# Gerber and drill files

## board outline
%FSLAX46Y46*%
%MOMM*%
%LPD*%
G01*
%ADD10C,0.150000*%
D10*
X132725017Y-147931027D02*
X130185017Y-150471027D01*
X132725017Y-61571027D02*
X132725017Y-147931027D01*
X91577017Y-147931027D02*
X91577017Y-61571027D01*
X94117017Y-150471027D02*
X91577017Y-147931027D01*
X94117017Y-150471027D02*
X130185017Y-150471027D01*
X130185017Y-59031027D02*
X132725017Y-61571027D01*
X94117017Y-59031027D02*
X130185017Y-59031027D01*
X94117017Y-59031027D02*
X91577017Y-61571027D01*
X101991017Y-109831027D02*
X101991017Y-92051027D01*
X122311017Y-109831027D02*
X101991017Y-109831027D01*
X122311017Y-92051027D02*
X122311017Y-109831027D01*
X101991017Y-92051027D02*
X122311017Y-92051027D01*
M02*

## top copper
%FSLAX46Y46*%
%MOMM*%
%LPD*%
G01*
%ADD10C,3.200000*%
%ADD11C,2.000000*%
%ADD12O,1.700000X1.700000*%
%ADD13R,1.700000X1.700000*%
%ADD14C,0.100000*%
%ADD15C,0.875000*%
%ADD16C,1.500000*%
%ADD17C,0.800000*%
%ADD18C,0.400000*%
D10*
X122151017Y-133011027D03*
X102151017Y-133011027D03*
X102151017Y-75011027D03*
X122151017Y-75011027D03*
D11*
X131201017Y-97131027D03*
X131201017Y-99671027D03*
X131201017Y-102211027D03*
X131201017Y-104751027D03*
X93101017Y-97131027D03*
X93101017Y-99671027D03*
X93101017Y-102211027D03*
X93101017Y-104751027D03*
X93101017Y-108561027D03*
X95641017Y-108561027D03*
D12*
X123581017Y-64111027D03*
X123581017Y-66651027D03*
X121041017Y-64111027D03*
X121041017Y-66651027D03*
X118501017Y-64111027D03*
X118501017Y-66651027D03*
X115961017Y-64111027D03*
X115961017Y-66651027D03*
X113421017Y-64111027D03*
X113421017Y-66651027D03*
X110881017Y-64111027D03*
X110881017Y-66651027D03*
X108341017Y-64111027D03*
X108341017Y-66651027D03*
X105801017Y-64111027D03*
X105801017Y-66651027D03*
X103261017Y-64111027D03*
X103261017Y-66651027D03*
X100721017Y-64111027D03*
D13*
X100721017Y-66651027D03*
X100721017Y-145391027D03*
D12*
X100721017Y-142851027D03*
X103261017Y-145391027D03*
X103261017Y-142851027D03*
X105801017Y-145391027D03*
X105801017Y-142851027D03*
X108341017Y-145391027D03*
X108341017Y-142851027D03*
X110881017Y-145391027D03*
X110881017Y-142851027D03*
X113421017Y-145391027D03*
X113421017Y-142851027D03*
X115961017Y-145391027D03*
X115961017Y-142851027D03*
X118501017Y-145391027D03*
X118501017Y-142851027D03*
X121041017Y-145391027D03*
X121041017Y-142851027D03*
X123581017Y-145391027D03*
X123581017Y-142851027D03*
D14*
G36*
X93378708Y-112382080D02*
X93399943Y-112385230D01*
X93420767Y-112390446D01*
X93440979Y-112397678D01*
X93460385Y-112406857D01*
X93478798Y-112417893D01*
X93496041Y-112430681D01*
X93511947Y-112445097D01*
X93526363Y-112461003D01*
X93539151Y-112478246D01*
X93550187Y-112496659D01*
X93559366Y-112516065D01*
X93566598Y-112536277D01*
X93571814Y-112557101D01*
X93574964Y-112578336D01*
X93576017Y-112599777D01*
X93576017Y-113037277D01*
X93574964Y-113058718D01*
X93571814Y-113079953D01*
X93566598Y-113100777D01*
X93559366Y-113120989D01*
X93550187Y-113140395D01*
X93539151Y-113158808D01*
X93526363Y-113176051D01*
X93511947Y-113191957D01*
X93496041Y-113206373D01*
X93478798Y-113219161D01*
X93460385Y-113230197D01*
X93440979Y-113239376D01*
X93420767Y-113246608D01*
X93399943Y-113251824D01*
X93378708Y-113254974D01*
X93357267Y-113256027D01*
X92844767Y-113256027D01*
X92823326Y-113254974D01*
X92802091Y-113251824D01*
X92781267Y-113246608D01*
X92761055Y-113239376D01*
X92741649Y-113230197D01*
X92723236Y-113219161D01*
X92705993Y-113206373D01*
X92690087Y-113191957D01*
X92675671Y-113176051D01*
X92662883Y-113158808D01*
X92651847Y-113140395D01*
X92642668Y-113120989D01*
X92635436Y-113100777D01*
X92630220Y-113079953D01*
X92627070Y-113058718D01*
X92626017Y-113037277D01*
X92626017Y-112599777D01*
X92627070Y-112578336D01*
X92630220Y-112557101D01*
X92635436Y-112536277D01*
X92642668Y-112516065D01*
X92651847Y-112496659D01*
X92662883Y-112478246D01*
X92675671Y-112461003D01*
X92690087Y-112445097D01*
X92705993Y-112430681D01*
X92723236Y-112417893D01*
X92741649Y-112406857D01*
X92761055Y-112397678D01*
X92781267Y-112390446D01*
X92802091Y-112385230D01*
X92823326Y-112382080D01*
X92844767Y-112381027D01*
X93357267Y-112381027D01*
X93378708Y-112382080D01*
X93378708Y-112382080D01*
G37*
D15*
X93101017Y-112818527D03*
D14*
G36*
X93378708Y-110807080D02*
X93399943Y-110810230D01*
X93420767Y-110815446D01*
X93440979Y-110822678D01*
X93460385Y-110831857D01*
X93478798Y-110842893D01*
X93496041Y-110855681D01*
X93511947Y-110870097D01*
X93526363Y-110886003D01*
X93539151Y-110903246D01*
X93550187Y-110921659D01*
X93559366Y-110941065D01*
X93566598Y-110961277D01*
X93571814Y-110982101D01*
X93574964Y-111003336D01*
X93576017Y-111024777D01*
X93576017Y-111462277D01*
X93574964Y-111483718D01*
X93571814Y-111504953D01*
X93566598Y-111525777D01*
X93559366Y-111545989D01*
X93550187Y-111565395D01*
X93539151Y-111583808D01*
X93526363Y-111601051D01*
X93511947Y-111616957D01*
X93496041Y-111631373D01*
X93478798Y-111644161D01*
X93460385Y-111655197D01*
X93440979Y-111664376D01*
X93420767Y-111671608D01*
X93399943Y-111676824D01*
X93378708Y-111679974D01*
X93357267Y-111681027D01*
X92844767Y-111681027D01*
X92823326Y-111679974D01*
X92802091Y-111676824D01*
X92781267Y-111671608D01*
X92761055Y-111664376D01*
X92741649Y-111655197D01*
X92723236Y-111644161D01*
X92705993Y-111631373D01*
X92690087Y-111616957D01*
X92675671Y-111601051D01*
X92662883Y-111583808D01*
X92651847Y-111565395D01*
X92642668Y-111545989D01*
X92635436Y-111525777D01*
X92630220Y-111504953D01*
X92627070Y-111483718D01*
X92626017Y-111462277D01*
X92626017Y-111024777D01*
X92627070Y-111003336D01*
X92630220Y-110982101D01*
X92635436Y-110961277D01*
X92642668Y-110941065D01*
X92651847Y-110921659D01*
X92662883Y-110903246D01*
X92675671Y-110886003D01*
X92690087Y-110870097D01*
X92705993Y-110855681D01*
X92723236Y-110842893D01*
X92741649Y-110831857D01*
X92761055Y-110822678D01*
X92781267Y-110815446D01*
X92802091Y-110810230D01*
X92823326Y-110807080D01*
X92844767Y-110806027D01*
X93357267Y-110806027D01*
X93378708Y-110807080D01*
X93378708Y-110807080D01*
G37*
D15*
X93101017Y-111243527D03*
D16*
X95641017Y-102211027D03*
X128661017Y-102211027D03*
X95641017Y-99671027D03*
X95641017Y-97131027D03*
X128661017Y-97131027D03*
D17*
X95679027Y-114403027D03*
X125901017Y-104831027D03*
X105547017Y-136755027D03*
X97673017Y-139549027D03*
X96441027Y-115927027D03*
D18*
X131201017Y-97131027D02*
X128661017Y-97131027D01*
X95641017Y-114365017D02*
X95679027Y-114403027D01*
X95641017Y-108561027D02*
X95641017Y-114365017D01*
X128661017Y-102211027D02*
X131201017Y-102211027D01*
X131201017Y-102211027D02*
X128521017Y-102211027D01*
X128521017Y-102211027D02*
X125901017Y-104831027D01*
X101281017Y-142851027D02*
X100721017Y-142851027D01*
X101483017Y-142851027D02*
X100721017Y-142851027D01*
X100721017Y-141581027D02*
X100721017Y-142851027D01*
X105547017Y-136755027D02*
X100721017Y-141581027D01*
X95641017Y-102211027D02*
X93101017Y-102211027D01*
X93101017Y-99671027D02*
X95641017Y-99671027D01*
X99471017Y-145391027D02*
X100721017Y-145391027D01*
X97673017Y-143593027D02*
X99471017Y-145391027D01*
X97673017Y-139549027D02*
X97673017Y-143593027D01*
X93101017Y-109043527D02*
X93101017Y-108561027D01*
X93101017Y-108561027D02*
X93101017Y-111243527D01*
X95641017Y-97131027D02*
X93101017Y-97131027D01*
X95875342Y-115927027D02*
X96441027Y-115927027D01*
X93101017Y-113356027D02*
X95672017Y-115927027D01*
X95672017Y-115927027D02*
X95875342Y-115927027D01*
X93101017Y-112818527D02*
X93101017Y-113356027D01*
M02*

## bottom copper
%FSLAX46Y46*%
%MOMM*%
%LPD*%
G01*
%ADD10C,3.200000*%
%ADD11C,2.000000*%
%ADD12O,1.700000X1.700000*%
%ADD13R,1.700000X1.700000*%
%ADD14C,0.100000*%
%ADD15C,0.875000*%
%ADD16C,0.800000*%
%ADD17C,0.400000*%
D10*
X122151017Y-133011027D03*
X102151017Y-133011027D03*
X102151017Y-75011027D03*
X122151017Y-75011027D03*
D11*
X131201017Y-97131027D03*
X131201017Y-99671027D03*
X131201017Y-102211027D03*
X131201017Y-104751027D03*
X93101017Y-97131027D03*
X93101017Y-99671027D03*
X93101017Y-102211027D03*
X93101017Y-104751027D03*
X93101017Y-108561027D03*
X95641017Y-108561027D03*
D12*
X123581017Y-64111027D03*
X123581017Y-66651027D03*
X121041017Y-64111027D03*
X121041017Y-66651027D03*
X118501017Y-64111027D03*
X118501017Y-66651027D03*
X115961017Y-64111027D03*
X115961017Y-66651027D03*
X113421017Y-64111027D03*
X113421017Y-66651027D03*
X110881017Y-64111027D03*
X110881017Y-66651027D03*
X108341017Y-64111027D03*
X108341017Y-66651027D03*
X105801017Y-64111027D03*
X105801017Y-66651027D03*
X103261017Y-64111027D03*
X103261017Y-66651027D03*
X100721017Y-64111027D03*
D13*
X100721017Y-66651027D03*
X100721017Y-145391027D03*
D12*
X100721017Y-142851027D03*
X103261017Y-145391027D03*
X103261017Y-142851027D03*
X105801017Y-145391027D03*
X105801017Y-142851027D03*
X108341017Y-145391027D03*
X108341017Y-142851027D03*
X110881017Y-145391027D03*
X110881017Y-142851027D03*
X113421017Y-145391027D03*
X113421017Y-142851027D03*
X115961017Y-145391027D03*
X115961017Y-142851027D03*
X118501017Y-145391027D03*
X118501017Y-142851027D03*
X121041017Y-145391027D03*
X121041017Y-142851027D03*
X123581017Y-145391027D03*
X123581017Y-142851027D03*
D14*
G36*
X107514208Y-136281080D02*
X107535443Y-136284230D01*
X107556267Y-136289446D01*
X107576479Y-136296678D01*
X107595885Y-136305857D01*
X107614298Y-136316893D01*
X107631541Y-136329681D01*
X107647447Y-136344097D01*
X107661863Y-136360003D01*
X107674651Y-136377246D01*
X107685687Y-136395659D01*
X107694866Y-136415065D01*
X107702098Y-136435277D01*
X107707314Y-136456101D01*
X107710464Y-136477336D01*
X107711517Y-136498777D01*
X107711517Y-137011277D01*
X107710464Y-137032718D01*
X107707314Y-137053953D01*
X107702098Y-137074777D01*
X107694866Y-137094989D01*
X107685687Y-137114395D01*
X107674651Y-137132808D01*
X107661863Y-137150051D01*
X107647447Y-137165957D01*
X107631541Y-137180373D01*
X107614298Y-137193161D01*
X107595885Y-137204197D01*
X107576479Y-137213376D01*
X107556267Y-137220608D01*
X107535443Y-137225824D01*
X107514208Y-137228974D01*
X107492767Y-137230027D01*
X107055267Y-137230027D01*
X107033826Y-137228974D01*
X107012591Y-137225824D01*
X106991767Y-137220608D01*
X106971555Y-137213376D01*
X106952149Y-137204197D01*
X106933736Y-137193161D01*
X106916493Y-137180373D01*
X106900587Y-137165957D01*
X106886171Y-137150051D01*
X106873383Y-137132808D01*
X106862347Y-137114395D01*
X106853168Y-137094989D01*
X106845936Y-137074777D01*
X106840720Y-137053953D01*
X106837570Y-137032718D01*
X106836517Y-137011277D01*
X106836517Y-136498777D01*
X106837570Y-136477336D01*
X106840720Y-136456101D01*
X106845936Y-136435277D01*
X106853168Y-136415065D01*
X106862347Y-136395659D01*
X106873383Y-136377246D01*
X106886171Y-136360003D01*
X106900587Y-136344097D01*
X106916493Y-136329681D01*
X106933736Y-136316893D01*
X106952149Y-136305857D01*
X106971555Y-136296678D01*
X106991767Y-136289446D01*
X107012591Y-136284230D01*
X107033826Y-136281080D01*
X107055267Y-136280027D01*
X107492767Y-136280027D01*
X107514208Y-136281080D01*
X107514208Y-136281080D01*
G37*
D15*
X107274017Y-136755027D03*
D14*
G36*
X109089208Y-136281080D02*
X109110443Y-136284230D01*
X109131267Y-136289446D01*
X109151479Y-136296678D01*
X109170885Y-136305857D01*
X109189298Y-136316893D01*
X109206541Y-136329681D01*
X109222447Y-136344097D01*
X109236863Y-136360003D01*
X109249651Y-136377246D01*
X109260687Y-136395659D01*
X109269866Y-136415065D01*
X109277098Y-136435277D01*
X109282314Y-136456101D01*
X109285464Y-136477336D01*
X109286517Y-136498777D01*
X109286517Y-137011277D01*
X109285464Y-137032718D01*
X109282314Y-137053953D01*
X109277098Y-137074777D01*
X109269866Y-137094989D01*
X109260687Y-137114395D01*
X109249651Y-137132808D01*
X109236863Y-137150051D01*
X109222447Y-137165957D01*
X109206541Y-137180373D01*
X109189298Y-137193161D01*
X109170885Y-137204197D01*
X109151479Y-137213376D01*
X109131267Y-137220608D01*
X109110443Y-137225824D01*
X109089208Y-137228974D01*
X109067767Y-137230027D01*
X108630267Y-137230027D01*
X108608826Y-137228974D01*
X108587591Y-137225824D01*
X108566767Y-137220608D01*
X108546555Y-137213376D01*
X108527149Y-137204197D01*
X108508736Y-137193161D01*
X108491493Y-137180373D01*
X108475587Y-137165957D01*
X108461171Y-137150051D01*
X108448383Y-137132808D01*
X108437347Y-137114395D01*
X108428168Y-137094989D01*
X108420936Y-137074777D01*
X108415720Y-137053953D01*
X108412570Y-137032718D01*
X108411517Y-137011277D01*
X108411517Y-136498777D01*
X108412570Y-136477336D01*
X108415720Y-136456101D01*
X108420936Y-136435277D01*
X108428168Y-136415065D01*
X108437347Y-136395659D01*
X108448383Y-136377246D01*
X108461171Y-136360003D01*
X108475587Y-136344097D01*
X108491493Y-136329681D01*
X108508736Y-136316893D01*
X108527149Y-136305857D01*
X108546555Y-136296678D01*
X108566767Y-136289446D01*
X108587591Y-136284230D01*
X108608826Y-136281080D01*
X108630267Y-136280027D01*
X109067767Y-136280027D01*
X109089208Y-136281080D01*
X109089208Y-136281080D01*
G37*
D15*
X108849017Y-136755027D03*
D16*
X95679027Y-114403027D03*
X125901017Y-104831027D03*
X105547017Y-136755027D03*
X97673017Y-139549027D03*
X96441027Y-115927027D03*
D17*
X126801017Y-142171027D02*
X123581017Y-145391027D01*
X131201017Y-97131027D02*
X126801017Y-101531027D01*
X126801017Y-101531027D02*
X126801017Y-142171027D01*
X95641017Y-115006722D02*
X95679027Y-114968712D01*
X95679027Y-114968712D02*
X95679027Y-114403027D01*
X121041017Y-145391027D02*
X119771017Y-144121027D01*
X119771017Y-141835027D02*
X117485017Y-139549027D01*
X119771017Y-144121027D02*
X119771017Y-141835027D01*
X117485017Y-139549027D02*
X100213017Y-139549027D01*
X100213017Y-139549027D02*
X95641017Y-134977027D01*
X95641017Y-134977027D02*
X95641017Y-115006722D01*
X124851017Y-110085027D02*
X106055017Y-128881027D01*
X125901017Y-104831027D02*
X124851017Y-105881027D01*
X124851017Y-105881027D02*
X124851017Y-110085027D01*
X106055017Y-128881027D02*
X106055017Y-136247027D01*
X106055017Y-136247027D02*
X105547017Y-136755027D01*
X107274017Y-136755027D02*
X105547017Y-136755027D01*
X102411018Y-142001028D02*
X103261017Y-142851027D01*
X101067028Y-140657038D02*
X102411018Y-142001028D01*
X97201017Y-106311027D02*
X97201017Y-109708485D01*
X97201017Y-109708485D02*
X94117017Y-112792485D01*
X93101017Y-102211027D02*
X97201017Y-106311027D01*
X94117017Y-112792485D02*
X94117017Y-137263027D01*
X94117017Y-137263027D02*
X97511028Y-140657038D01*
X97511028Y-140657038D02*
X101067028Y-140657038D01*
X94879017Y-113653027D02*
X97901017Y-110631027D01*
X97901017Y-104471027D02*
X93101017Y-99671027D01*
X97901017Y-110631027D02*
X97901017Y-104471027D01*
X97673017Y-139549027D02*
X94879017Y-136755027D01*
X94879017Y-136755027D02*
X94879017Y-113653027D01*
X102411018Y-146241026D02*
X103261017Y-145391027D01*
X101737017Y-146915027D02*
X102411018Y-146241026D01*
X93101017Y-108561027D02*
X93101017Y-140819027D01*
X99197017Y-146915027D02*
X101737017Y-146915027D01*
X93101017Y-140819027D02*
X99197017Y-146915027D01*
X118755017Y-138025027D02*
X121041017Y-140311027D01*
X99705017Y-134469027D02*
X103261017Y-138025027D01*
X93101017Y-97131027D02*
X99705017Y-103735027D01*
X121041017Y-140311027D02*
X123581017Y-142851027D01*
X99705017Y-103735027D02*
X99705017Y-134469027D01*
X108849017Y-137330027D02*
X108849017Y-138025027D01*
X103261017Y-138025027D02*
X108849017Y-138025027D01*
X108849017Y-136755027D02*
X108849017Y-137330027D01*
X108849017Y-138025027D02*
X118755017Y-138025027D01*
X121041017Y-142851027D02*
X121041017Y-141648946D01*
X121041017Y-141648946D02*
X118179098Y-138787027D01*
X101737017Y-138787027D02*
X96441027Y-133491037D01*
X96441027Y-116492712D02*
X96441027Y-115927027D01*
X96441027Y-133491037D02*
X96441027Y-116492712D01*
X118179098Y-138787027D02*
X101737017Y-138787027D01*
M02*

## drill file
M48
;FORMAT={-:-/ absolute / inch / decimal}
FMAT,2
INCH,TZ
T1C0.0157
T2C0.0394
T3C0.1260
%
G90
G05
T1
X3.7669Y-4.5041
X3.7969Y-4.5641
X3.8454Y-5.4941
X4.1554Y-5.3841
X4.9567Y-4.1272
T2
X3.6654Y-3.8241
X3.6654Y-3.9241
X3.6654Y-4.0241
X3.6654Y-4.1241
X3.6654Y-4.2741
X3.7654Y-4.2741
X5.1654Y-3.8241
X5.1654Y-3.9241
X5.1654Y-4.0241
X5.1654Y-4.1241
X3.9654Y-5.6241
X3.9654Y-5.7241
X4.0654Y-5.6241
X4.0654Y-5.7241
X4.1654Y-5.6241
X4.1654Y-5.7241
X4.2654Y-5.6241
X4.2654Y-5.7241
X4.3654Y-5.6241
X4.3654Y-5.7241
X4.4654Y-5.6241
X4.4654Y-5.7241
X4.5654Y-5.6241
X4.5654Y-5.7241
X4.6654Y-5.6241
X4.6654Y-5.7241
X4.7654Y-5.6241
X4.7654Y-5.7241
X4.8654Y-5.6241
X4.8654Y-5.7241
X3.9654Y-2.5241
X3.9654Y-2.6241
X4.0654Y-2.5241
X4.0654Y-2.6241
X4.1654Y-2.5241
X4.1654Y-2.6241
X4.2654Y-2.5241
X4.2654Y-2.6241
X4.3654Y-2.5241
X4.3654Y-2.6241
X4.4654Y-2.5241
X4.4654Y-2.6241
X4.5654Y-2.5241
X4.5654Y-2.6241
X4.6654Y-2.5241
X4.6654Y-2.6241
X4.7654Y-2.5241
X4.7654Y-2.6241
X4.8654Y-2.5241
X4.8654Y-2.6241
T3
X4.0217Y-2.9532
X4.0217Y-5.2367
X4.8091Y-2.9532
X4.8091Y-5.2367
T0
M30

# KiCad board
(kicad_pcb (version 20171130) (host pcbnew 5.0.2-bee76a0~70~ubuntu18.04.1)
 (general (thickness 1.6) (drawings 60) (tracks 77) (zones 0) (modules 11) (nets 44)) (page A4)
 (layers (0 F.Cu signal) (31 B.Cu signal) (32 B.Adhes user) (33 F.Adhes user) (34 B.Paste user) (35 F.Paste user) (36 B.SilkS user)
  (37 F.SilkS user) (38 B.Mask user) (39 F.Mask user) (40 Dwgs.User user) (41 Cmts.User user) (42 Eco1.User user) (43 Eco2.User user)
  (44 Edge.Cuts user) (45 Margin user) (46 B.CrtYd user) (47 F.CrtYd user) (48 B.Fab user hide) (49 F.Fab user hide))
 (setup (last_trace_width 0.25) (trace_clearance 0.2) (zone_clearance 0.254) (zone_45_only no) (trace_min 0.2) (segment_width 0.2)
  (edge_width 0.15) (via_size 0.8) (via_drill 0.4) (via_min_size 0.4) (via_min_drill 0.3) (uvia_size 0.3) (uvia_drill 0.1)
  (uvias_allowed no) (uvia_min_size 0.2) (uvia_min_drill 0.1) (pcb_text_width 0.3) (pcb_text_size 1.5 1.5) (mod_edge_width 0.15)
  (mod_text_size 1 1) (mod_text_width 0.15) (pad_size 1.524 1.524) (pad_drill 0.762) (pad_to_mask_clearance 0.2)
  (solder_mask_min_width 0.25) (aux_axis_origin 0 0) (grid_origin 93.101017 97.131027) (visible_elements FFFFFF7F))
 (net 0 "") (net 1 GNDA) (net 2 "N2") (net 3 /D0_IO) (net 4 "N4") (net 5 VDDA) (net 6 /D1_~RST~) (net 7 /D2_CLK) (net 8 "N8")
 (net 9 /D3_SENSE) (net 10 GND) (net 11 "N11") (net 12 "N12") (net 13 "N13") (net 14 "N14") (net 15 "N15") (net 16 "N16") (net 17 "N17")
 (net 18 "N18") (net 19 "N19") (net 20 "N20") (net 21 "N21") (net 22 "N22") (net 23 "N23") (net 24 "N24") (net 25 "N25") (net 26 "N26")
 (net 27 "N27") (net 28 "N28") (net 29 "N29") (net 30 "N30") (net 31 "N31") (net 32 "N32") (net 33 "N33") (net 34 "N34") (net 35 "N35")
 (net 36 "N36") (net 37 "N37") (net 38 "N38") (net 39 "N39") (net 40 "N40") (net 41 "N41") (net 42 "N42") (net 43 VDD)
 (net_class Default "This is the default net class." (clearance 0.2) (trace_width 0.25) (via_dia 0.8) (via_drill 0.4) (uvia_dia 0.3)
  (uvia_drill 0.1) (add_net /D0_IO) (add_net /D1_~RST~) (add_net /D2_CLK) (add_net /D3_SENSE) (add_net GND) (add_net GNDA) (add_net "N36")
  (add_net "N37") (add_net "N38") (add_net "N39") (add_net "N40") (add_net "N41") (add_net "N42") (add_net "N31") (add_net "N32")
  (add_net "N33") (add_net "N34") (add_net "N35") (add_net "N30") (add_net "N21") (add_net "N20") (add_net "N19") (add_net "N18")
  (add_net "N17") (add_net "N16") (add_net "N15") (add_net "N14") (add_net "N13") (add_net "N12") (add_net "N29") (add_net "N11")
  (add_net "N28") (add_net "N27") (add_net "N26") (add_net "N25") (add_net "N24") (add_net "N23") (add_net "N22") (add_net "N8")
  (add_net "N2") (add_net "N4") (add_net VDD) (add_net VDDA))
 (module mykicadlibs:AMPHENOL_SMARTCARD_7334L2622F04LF (layer B.Cu) (at 112.151017 104.011027 270)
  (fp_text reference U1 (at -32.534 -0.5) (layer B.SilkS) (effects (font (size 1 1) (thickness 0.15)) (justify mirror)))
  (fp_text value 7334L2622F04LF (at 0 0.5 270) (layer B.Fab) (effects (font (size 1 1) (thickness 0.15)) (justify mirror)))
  (pad ~ thru_hole circle (at 29 -10 270) (size 3.2 3.2) (drill 3.2) (layers *.Cu *.Mask))
  (pad ~ thru_hole circle (at 29 10 270) (size 3.2 3.2) (drill 3.2) (layers *.Cu *.Mask))
  (pad ~ thru_hole circle (at -29 10 270) (size 3.2 3.2) (drill 3.2) (layers *.Cu *.Mask))
  (pad ~ thru_hole circle (at -29 -10 270) (size 3.2 3.2) (drill 3.2) (layers *.Cu *.Mask))
  (pad 5 thru_hole circle (at -6.88 -19.05 270) (size 2 2) (drill 1) (layers *.Cu *.Mask) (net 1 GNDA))
  (pad 6 thru_hole circle (at -4.34 -19.05 270) (size 2 2) (drill 1) (layers *.Cu *.Mask) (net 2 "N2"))
  (pad 7 thru_hole circle (at -1.8 -19.05 270) (size 2 2) (drill 1) (layers *.Cu *.Mask) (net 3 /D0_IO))
  (pad 8 thru_hole circle (at 0.74 -19.05 270) (size 2 2) (drill 1) (layers *.Cu *.Mask) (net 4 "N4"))
  (pad 1 thru_hole circle (at -6.88 19.05 270) (size 2 2) (drill 1) (layers *.Cu *.Mask) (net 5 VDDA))
  (pad 2 thru_hole circle (at -4.34 19.05 270) (size 2 2) (drill 1) (layers *.Cu *.Mask) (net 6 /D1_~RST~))
  (pad 3 thru_hole circle (at -1.8 19.05 270) (size 2 2) (drill 1) (layers *.Cu *.Mask) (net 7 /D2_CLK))
  (pad 4 thru_hole circle (at 0.74 19.05 270) (size 2 2) (drill 1) (layers *.Cu *.Mask) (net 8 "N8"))
  (pad 9 thru_hole circle (at 4.55 19.05 270) (size 2 2) (drill 1) (layers *.Cu *.Mask) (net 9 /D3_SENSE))
  (pad 10 thru_hole circle (at 4.55 16.51 270) (size 2 2) (drill 1) (layers *.Cu *.Mask) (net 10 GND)))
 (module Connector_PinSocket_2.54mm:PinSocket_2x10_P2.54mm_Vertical (layer B.Cu) (at 100.721017 66.651027 270)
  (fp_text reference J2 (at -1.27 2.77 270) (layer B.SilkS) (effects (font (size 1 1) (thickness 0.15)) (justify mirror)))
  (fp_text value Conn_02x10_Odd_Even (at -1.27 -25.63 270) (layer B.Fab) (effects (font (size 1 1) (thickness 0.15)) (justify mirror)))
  (pad 20 thru_hole oval (at -2.54 -22.86 270) (size 1.7 1.7) (drill 1) (layers *.Cu *.Mask) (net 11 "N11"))
  (pad 19 thru_hole oval (at 0 -22.86 270) (size 1.7 1.7) (drill 1) (layers *.Cu *.Mask) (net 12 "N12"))
  (pad 18 thru_hole oval (at -2.54 -20.32 270) (size 1.7 1.7) (drill 1) (layers *.Cu *.Mask) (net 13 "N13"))
  (pad 17 thru_hole oval (at 0 -20.32 270) (size 1.7 1.7) (drill 1) (layers *.Cu *.Mask) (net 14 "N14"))
  (pad 16 thru_hole oval (at -2.54 -17.78 270) (size 1.7 1.7) (drill 1) (layers *.Cu *.Mask) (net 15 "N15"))
  (pad 15 thru_hole oval (at 0 -17.78 270) (size 1.7 1.7) (drill 1) (layers *.Cu *.Mask) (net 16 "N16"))
  (pad 14 thru_hole oval (at -2.54 -15.24 270) (size 1.7 1.7) (drill 1) (layers *.Cu *.Mask) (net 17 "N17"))
  (pad 13 thru_hole oval (at 0 -15.24 270) (size 1.7 1.7) (drill 1) (layers *.Cu *.Mask) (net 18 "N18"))
  (pad 12 thru_hole oval (at -2.54 -12.7 270) (size 1.7 1.7) (drill 1) (layers *.Cu *.Mask) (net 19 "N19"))
  (pad 11 thru_hole oval (at 0 -12.7 270) (size 1.7 1.7) (drill 1) (layers *.Cu *.Mask) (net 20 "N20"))
  (pad 10 thru_hole oval (at -2.54 -10.16 270) (size 1.7 1.7) (drill 1) (layers *.Cu *.Mask) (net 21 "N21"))
  (pad 9 thru_hole oval (at 0 -10.16 270) (size 1.7 1.7) (drill 1) (layers *.Cu *.Mask) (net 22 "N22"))
  (pad 8 thru_hole oval (at -2.54 -7.62 270) (size 1.7 1.7) (drill 1) (layers *.Cu *.Mask) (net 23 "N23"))
  (pad 7 thru_hole oval (at 0 -7.62 270) (size 1.7 1.7) (drill 1) (layers *.Cu *.Mask) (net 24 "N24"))
  (pad 6 thru_hole oval (at -2.54 -5.08 270) (size 1.7 1.7) (drill 1) (layers *.Cu *.Mask) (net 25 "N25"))
  (pad 5 thru_hole oval (at 0 -5.08 270) (size 1.7 1.7) (drill 1) (layers *.Cu *.Mask) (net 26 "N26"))
  (pad 4 thru_hole oval (at -2.54 -2.54 270) (size 1.7 1.7) (drill 1) (layers *.Cu *.Mask) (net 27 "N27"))
  (pad 3 thru_hole oval (at 0 -2.54 270) (size 1.7 1.7) (drill 1) (layers *.Cu *.Mask) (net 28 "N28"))
  (pad 2 thru_hole oval (at -2.54 0 270) (size 1.7 1.7) (drill 1) (layers *.Cu *.Mask) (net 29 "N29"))
  (pad 1 thru_hole rect (at 0 0 270) (size 1.7 1.7) (drill 1) (layers *.Cu *.Mask) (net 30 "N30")))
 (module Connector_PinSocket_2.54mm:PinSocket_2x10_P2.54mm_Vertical (layer B.Cu) (at 100.721017 145.391027 270)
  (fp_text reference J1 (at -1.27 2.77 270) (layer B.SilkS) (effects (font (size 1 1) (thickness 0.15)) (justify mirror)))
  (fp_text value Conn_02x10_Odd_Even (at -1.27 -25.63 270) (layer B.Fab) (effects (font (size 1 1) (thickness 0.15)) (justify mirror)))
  (pad 1 thru_hole rect (at 0 0 270) (size 1.7 1.7) (drill 1) (layers *.Cu *.Mask) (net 6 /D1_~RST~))
  (pad 2 thru_hole oval (at -2.54 0 270) (size 1.7 1.7) (drill 1) (layers *.Cu *.Mask) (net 3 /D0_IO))
  (pad 3 thru_hole oval (at 0 -2.54 270) (size 1.7 1.7) (drill 1) (layers *.Cu *.Mask) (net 9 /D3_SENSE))
  (pad 4 thru_hole oval (at -2.54 -2.54 270) (size 1.7 1.7) (drill 1) (layers *.Cu *.Mask) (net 7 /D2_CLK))
  (pad 5 thru_hole oval (at 0 -5.08 270) (size 1.7 1.7) (drill 1) (layers *.Cu *.Mask) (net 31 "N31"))
  (pad 6 thru_hole oval (at -2.54 -5.08 270) (size 1.7 1.7) (drill 1) (layers *.Cu *.Mask) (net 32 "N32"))
  (pad 7 thru_hole oval (at 0 -7.62 270) (size 1.7 1.7) (drill 1) (layers *.Cu *.Mask) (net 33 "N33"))
  (pad 8 thru_hole oval (at -2.54 -7.62 270) (size 1.7 1.7) (drill 1) (layers *.Cu *.Mask) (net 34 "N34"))
  (pad 9 thru_hole oval (at 0 -10.16 270) (size 1.7 1.7) (drill 1) (layers *.Cu *.Mask) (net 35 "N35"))
  (pad 10 thru_hole oval (at -2.54 -10.16 270) (size 1.7 1.7) (drill 1) (layers *.Cu *.Mask) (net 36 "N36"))
  (pad 11 thru_hole oval (at 0 -12.7 270) (size 1.7 1.7) (drill 1) (layers *.Cu *.Mask) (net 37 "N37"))
  (pad 12 thru_hole oval (at -2.54 -12.7 270) (size 1.7 1.7) (drill 1) (layers *.Cu *.Mask) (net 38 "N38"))
  (pad 13 thru_hole oval (at 0 -15.24 270) (size 1.7 1.7) (drill 1) (layers *.Cu *.Mask) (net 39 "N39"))
  (pad 14 thru_hole oval (at -2.54 -15.24 270) (size 1.7 1.7) (drill 1) (layers *.Cu *.Mask) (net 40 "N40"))
  (pad 15 thru_hole oval (at 0 -17.78 270) (size 1.7 1.7) (drill 1) (layers *.Cu *.Mask) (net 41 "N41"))
  (pad 16 thru_hole oval (at -2.54 -17.78 270) (size 1.7 1.7) (drill 1) (layers *.Cu *.Mask) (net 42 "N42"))
  (pad 17 thru_hole oval (at 0 -20.32 270) (size 1.7 1.7) (drill 1) (layers *.Cu *.Mask) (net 10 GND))
  (pad 18 thru_hole oval (at -2.54 -20.32 270) (size 1.7 1.7) (drill 1) (layers *.Cu *.Mask) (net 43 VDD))
  (pad 19 thru_hole oval (at 0 -22.86 270) (size 1.7 1.7) (drill 1) (layers *.Cu *.Mask) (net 1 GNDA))
  (pad 20 thru_hole oval (at -2.54 -22.86 270) (size 1.7 1.7) (drill 1) (layers *.Cu *.Mask) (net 5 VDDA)))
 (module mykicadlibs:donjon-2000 (layer F.Cu) (at 95.641017 65.127027)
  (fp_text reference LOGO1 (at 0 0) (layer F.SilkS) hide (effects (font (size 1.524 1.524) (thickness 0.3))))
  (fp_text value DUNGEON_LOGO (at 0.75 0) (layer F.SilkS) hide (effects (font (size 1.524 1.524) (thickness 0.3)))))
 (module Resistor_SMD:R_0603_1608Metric (layer B.Cu) (at 108.061517 136.755027)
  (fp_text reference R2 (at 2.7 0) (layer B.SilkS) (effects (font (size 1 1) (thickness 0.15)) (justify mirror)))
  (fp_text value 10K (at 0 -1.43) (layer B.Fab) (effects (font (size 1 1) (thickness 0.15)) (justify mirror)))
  (pad 1 smd roundrect (at -0.7875 0) (size 0.875 0.95) (layers B.Cu B.Paste B.Mask) (roundrect_rratio 0.25) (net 3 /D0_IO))
  (pad 2 smd roundrect (at 0.7875 0) (size 0.875 0.95) (layers B.Cu B.Paste B.Mask) (roundrect_rratio 0.25) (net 5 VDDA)))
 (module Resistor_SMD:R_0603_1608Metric (layer F.Cu) (at 93.101017 112.031027 90)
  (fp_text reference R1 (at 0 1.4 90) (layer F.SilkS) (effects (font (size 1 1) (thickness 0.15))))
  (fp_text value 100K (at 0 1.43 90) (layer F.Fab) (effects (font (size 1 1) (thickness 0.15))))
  (pad 1 smd roundrect (at -0.7875 0 90) (size 0.875 0.95) (layers F.Cu F.Paste F.Mask) (roundrect_rratio 0.25) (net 43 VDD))
  (pad 2 smd roundrect (at 0.7875 0 90) (size 0.875 0.95) (layers F.Cu F.Paste F.Mask) (roundrect_rratio 0.25) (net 9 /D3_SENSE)))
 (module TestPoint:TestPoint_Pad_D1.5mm (layer F.Cu) (at 95.641017 102.211027)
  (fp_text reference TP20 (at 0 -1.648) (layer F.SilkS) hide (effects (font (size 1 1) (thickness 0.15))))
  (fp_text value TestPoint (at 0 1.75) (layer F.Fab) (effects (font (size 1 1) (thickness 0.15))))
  (pad 1 smd circle (at 0 0) (size 1.5 1.5) (layers F.Cu F.Mask) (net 7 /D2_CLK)))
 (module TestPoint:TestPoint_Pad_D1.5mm (layer F.Cu) (at 128.661017 102.211027)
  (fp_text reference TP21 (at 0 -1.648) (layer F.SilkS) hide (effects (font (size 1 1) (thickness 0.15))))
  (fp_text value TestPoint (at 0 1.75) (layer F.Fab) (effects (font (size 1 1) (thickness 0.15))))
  (pad 1 smd circle (at 0 0) (size 1.5 1.5) (layers F.Cu F.Mask) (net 3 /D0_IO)))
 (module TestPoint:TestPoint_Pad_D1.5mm (layer F.Cu) (at 95.641017 99.671027)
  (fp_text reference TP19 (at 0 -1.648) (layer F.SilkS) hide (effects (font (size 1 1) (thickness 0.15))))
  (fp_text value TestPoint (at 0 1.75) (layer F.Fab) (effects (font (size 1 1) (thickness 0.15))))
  (pad 1 smd circle (at 0 0) (size 1.5 1.5) (layers F.Cu F.Mask) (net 6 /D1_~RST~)))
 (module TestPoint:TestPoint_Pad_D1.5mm (layer F.Cu) (at 95.641017 97.131027)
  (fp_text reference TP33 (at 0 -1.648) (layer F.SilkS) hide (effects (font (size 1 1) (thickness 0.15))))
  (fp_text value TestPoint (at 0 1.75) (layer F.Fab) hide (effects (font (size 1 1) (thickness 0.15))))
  (pad 1 smd circle (at 0 0) (size 1.5 1.5) (layers F.Cu F.Mask) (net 5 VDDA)))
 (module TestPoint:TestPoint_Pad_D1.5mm (layer F.Cu) (at 128.661017 97.131027)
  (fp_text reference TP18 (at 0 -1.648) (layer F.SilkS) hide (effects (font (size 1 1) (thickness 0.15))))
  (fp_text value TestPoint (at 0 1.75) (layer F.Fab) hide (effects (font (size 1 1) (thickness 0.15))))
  (pad 1 smd circle (at 0 0) (size 1.5 1.5) (layers F.Cu F.Mask) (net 1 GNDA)))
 (gr_line (start 132.725017 147.931027) (end 130.185017 150.471027) (layer Edge.Cuts) (width 0.15))
 (gr_line (start 132.725017 61.571027) (end 132.725017 147.931027) (layer Edge.Cuts) (width 0.15))
 (gr_line (start 91.577017 147.931027) (end 91.577017 61.571027) (layer Edge.Cuts) (width 0.15))
 (gr_line (start 94.117017 150.471027) (end 91.577017 147.931027) (layer Edge.Cuts) (width 0.15))
 (gr_line (start 94.117017 150.471027) (end 130.185017 150.471027) (layer Edge.Cuts) (width 0.15))
 (gr_line (start 130.185017 59.031027) (end 132.725017 61.571027) (layer Edge.Cuts) (width 0.15))
 (gr_line (start 94.117017 59.031027) (end 130.185017 59.031027) (layer Edge.Cuts) (width 0.15))
 (gr_line (start 94.117017 59.031027) (end 91.577017 61.571027) (layer Edge.Cuts) (width 0.15))
 (gr_line (start 101.991017 109.831027) (end 101.991017 92.051027) (layer Edge.Cuts) (width 0.15))
 (gr_line (start 122.311017 109.831027) (end 101.991017 109.831027) (layer Edge.Cuts) (width 0.15))
 (gr_line (start 122.311017 92.051027) (end 122.311017 109.831027) (layer Edge.Cuts) (width 0.15))
 (gr_line (start 101.991017 92.051027) (end 122.311017 92.051027) (layer Edge.Cuts) (width 0.15))
 (segment (start 131.201017 97.131027) (end 128.661017 97.131027) (width 0.4) (layer F.Cu) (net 1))
 (segment (start 126.801017 142.171027) (end 123.581017 145.391027) (width 0.4) (layer B.Cu) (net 1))
 (segment (start 131.201017 97.131027) (end 126.801017 101.531027) (width 0.4) (layer B.Cu) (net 1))
 (segment (start 126.801017 101.531027) (end 126.801017 142.171027) (width 0.4) (layer B.Cu) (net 1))
 (via (at 95.679027 114.403027) (size 0.8) (drill 0.4) (layers F.Cu B.Cu) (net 10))
 (segment (start 95.641017 114.365017) (end 95.679027 114.403027) (width 0.4) (layer F.Cu) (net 10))
 (segment (start 95.641017 108.561027) (end 95.641017 114.365017) (width 0.4) (layer F.Cu) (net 10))
 (segment (start 95.641017 115.006722) (end 95.679027 114.968712) (width 0.4) (layer B.Cu) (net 10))
 (segment (start 95.679027 114.968712) (end 95.679027 114.403027) (width 0.4) (layer B.Cu) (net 10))
 (segment (start 121.041017 145.391027) (end 119.771017 144.121027) (width 0.4) (layer B.Cu) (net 10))
 (segment (start 119.771017 141.835027) (end 117.485017 139.549027) (width 0.4) (layer B.Cu) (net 10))
 (segment (start 119.771017 144.121027) (end 119.771017 141.835027) (width 0.4) (layer B.Cu) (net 10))
 (segment (start 117.485017 139.549027) (end 100.213017 139.549027) (width 0.4) (layer B.Cu) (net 10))
 (segment (start 100.213017 139.549027) (end 95.641017 134.977027) (width 0.4) (layer B.Cu) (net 10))
 (segment (start 95.641017 134.977027) (end 95.641017 115.006722) (width 0.4) (layer B.Cu) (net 10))
 (segment (start 128.661017 102.211027) (end 131.201017 102.211027) (width 0.4) (layer F.Cu) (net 3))
 (via (at 125.901017 104.831027) (size 0.8) (drill 0.4) (layers F.Cu B.Cu) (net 3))
 (segment (start 131.201017 102.211027) (end 128.521017 102.211027) (width 0.4) (layer F.Cu) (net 3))
 (segment (start 128.521017 102.211027) (end 125.901017 104.831027) (width 0.4) (layer F.Cu) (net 3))
 (segment (start 124.851017 110.085027) (end 106.055017 128.881027) (width 0.4) (layer B.Cu) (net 3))
 (segment (start 125.901017 104.831027) (end 124.851017 105.881027) (width 0.4) (layer B.Cu) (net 3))
 (segment (start 124.851017 105.881027) (end 124.851017 110.085027) (width 0.4) (layer B.Cu) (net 3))
 (segment (start 101.281017 142.851027) (end 100.721017 142.851027) (width 0.4) (layer F.Cu) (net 3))
 (segment (start 101.483017 142.851027) (end 100.721017 142.851027) (width 0.4) (layer F.Cu) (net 3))
 (via (at 105.547017 136.755027) (size 0.8) (drill 0.4) (layers F.Cu B.Cu) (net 3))
 (segment (start 106.055017 128.881027) (end 106.055017 136.247027) (width 0.4) (layer B.Cu) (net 3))
 (segment (start 106.055017 136.247027) (end 105.547017 136.755027) (width 0.4) (layer B.Cu) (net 3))
 (segment (start 100.721017 141.581027) (end 100.721017 142.851027) (width 0.4) (layer F.Cu) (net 3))
 (segment (start 105.547017 136.755027) (end 100.721017 141.581027) (width 0.4) (layer F.Cu) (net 3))
 (segment (start 107.274017 136.755027) (end 105.547017 136.755027) (width 0.4) (layer B.Cu) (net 3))
 (segment (start 95.641017 102.211027) (end 93.101017 102.211027) (width 0.4) (layer F.Cu) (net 7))
 (segment (start 102.411018 142.001028) (end 103.261017 142.851027) (width 0.4) (layer B.Cu) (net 7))
 (segment (start 101.067028 140.657038) (end 102.411018 142.001028) (width 0.4) (layer B.Cu) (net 7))
 (segment (start 97.201017 106.311027) (end 97.201017 109.708485) (width 0.4) (layer B.Cu) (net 7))
 (segment (start 97.201017 109.708485) (end 94.117017 112.792485) (width 0.4) (layer B.Cu) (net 7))
 (segment (start 93.101017 102.211027) (end 97.201017 106.311027) (width 0.4) (layer B.Cu) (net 7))
 (segment (start 94.117017 112.792485) (end 94.117017 137.263027) (width 0.4) (layer B.Cu) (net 7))
 (segment (start 94.117017 137.263027) (end 97.511028 140.657038) (width 0.4) (layer B.Cu) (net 7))
 (segment (start 97.511028 140.657038) (end 101.067028 140.657038) (width 0.4) (layer B.Cu) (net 7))
 (segment (start 93.101017 99.671027) (end 95.641017 99.671027) (width 0.4) (layer F.Cu) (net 6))
 (via (at 97.673017 139.549027) (size 0.8) (drill 0.4) (layers F.Cu B.Cu) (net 6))
 (segment (start 99.471017 145.391027) (end 100.721017 145.391027) (width 0.4) (layer F.Cu) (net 6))
 (segment (start 97.673017 143.593027) (end 99.471017 145.391027) (width 0.4) (layer F.Cu) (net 6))
 (segment (start 97.673017 139.549027) (end 97.673017 143.593027) (width 0.4) (layer F.Cu) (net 6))
 (segment (start 94.879017 113.653027) (end 97.901017 110.631027) (width 0.4) (layer B.Cu) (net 6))
 (segment (start 97.901017 104.471027) (end 93.101017 99.671027) (width 0.4) (layer B.Cu) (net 6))
 (segment (start 97.901017 110.631027) (end 97.901017 104.471027) (width 0.4) (layer B.Cu) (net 6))
 (segment (start 97.673017 139.549027) (end 94.879017 136.755027) (width 0.4) (layer B.Cu) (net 6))
 (segment (start 94.879017 136.755027) (end 94.879017 113.653027) (width 0.4) (layer B.Cu) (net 6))
 (segment (start 93.101017 109.043527) (end 93.101017 108.561027) (width 0.4) (layer F.Cu) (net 9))
 (segment (start 93.101017 108.561027) (end 93.101017 111.243527) (width 0.4) (layer F.Cu) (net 9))
 (segment (start 102.411018 146.241026) (end 103.261017 145.391027) (width 0.4) (layer B.Cu) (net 9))
 (segment (start 101.737017 146.915027) (end 102.411018 146.241026) (width 0.4) (layer B.Cu) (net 9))
 (segment (start 93.101017 108.561027) (end 93.101017 140.819027) (width 0.4) (layer B.Cu) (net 9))
 (segment (start 99.197017 146.915027) (end 101.737017 146.915027) (width 0.4) (layer B.Cu) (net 9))
 (segment (start 93.101017 140.819027) (end 99.197017 146.915027) (width 0.4) (layer B.Cu) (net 9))
 (segment (start 95.641017 97.131027) (end 93.101017 97.131027) (width 0.4) (layer F.Cu) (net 5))
 (segment (start 118.755017 138.025027) (end 121.041017 140.311027) (width 0.4) (layer B.Cu) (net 5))
 (segment (start 99.705017 134.469027) (end 103.261017 138.025027) (width 0.4) (layer B.Cu) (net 5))
 (segment (start 93.101017 97.131027) (end 99.705017 103.735027) (width 0.4) (layer B.Cu) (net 5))
 (segment (start 121.041017 140.311027) (end 123.581017 142.851027) (width 0.4) (layer B.Cu) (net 5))
 (segment (start 99.705017 103.735027) (end 99.705017 134.469027) (width 0.4) (layer B.Cu) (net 5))
 (segment (start 108.849017 137.330027) (end 108.849017 138.025027) (width 0.4) (layer B.Cu) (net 5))
 (segment (start 103.261017 138.025027) (end 108.849017 138.025027) (width 0.4) (layer B.Cu) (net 5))
 (segment (start 108.849017 136.755027) (end 108.849017 137.330027) (width 0.4) (layer B.Cu) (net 5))
 (segment (start 108.849017 138.025027) (end 118.755017 138.025027) (width 0.4) (layer B.Cu) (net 5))
 (segment (start 95.875342 115.927027) (end 96.441027 115.927027) (width 0.4) (layer F.Cu) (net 43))
 (segment (start 121.041017 142.851027) (end 121.041017 141.648946) (width 0.4) (layer B.Cu) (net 43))
 (segment (start 121.041017 141.648946) (end 118.179098 138.787027) (width 0.4) (layer B.Cu) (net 43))
 (segment (start 101.737017 138.787027) (end 96.441027 133.491037) (width 0.4) (layer B.Cu) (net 43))
 (segment (start 96.441027 116.492712) (end 96.441027 115.927027) (width 0.4) (layer B.Cu) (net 43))
 (segment (start 96.441027 133.491037) (end 96.441027 116.492712) (width 0.4) (layer B.Cu) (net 43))
 (segment (start 93.101017 113.356027) (end 95.672017 115.927027) (width 0.4) (layer F.Cu) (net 43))
 (segment (start 118.179098 138.787027) (end 101.737017 138.787027) (width 0.4) (layer B.Cu) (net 43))
 (segment (start 95.672017 115.927027) (end 95.875342 115.927027) (width 0.4) (layer F.Cu) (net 43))
 (segment (start 93.101017 112.818527) (end 93.101017 113.356027) (width 0.4) (layer F.Cu) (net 43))
 (via (at 96.441027 115.927027) (size 0.8) (drill 0.4) (layers F.Cu B.Cu) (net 43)))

